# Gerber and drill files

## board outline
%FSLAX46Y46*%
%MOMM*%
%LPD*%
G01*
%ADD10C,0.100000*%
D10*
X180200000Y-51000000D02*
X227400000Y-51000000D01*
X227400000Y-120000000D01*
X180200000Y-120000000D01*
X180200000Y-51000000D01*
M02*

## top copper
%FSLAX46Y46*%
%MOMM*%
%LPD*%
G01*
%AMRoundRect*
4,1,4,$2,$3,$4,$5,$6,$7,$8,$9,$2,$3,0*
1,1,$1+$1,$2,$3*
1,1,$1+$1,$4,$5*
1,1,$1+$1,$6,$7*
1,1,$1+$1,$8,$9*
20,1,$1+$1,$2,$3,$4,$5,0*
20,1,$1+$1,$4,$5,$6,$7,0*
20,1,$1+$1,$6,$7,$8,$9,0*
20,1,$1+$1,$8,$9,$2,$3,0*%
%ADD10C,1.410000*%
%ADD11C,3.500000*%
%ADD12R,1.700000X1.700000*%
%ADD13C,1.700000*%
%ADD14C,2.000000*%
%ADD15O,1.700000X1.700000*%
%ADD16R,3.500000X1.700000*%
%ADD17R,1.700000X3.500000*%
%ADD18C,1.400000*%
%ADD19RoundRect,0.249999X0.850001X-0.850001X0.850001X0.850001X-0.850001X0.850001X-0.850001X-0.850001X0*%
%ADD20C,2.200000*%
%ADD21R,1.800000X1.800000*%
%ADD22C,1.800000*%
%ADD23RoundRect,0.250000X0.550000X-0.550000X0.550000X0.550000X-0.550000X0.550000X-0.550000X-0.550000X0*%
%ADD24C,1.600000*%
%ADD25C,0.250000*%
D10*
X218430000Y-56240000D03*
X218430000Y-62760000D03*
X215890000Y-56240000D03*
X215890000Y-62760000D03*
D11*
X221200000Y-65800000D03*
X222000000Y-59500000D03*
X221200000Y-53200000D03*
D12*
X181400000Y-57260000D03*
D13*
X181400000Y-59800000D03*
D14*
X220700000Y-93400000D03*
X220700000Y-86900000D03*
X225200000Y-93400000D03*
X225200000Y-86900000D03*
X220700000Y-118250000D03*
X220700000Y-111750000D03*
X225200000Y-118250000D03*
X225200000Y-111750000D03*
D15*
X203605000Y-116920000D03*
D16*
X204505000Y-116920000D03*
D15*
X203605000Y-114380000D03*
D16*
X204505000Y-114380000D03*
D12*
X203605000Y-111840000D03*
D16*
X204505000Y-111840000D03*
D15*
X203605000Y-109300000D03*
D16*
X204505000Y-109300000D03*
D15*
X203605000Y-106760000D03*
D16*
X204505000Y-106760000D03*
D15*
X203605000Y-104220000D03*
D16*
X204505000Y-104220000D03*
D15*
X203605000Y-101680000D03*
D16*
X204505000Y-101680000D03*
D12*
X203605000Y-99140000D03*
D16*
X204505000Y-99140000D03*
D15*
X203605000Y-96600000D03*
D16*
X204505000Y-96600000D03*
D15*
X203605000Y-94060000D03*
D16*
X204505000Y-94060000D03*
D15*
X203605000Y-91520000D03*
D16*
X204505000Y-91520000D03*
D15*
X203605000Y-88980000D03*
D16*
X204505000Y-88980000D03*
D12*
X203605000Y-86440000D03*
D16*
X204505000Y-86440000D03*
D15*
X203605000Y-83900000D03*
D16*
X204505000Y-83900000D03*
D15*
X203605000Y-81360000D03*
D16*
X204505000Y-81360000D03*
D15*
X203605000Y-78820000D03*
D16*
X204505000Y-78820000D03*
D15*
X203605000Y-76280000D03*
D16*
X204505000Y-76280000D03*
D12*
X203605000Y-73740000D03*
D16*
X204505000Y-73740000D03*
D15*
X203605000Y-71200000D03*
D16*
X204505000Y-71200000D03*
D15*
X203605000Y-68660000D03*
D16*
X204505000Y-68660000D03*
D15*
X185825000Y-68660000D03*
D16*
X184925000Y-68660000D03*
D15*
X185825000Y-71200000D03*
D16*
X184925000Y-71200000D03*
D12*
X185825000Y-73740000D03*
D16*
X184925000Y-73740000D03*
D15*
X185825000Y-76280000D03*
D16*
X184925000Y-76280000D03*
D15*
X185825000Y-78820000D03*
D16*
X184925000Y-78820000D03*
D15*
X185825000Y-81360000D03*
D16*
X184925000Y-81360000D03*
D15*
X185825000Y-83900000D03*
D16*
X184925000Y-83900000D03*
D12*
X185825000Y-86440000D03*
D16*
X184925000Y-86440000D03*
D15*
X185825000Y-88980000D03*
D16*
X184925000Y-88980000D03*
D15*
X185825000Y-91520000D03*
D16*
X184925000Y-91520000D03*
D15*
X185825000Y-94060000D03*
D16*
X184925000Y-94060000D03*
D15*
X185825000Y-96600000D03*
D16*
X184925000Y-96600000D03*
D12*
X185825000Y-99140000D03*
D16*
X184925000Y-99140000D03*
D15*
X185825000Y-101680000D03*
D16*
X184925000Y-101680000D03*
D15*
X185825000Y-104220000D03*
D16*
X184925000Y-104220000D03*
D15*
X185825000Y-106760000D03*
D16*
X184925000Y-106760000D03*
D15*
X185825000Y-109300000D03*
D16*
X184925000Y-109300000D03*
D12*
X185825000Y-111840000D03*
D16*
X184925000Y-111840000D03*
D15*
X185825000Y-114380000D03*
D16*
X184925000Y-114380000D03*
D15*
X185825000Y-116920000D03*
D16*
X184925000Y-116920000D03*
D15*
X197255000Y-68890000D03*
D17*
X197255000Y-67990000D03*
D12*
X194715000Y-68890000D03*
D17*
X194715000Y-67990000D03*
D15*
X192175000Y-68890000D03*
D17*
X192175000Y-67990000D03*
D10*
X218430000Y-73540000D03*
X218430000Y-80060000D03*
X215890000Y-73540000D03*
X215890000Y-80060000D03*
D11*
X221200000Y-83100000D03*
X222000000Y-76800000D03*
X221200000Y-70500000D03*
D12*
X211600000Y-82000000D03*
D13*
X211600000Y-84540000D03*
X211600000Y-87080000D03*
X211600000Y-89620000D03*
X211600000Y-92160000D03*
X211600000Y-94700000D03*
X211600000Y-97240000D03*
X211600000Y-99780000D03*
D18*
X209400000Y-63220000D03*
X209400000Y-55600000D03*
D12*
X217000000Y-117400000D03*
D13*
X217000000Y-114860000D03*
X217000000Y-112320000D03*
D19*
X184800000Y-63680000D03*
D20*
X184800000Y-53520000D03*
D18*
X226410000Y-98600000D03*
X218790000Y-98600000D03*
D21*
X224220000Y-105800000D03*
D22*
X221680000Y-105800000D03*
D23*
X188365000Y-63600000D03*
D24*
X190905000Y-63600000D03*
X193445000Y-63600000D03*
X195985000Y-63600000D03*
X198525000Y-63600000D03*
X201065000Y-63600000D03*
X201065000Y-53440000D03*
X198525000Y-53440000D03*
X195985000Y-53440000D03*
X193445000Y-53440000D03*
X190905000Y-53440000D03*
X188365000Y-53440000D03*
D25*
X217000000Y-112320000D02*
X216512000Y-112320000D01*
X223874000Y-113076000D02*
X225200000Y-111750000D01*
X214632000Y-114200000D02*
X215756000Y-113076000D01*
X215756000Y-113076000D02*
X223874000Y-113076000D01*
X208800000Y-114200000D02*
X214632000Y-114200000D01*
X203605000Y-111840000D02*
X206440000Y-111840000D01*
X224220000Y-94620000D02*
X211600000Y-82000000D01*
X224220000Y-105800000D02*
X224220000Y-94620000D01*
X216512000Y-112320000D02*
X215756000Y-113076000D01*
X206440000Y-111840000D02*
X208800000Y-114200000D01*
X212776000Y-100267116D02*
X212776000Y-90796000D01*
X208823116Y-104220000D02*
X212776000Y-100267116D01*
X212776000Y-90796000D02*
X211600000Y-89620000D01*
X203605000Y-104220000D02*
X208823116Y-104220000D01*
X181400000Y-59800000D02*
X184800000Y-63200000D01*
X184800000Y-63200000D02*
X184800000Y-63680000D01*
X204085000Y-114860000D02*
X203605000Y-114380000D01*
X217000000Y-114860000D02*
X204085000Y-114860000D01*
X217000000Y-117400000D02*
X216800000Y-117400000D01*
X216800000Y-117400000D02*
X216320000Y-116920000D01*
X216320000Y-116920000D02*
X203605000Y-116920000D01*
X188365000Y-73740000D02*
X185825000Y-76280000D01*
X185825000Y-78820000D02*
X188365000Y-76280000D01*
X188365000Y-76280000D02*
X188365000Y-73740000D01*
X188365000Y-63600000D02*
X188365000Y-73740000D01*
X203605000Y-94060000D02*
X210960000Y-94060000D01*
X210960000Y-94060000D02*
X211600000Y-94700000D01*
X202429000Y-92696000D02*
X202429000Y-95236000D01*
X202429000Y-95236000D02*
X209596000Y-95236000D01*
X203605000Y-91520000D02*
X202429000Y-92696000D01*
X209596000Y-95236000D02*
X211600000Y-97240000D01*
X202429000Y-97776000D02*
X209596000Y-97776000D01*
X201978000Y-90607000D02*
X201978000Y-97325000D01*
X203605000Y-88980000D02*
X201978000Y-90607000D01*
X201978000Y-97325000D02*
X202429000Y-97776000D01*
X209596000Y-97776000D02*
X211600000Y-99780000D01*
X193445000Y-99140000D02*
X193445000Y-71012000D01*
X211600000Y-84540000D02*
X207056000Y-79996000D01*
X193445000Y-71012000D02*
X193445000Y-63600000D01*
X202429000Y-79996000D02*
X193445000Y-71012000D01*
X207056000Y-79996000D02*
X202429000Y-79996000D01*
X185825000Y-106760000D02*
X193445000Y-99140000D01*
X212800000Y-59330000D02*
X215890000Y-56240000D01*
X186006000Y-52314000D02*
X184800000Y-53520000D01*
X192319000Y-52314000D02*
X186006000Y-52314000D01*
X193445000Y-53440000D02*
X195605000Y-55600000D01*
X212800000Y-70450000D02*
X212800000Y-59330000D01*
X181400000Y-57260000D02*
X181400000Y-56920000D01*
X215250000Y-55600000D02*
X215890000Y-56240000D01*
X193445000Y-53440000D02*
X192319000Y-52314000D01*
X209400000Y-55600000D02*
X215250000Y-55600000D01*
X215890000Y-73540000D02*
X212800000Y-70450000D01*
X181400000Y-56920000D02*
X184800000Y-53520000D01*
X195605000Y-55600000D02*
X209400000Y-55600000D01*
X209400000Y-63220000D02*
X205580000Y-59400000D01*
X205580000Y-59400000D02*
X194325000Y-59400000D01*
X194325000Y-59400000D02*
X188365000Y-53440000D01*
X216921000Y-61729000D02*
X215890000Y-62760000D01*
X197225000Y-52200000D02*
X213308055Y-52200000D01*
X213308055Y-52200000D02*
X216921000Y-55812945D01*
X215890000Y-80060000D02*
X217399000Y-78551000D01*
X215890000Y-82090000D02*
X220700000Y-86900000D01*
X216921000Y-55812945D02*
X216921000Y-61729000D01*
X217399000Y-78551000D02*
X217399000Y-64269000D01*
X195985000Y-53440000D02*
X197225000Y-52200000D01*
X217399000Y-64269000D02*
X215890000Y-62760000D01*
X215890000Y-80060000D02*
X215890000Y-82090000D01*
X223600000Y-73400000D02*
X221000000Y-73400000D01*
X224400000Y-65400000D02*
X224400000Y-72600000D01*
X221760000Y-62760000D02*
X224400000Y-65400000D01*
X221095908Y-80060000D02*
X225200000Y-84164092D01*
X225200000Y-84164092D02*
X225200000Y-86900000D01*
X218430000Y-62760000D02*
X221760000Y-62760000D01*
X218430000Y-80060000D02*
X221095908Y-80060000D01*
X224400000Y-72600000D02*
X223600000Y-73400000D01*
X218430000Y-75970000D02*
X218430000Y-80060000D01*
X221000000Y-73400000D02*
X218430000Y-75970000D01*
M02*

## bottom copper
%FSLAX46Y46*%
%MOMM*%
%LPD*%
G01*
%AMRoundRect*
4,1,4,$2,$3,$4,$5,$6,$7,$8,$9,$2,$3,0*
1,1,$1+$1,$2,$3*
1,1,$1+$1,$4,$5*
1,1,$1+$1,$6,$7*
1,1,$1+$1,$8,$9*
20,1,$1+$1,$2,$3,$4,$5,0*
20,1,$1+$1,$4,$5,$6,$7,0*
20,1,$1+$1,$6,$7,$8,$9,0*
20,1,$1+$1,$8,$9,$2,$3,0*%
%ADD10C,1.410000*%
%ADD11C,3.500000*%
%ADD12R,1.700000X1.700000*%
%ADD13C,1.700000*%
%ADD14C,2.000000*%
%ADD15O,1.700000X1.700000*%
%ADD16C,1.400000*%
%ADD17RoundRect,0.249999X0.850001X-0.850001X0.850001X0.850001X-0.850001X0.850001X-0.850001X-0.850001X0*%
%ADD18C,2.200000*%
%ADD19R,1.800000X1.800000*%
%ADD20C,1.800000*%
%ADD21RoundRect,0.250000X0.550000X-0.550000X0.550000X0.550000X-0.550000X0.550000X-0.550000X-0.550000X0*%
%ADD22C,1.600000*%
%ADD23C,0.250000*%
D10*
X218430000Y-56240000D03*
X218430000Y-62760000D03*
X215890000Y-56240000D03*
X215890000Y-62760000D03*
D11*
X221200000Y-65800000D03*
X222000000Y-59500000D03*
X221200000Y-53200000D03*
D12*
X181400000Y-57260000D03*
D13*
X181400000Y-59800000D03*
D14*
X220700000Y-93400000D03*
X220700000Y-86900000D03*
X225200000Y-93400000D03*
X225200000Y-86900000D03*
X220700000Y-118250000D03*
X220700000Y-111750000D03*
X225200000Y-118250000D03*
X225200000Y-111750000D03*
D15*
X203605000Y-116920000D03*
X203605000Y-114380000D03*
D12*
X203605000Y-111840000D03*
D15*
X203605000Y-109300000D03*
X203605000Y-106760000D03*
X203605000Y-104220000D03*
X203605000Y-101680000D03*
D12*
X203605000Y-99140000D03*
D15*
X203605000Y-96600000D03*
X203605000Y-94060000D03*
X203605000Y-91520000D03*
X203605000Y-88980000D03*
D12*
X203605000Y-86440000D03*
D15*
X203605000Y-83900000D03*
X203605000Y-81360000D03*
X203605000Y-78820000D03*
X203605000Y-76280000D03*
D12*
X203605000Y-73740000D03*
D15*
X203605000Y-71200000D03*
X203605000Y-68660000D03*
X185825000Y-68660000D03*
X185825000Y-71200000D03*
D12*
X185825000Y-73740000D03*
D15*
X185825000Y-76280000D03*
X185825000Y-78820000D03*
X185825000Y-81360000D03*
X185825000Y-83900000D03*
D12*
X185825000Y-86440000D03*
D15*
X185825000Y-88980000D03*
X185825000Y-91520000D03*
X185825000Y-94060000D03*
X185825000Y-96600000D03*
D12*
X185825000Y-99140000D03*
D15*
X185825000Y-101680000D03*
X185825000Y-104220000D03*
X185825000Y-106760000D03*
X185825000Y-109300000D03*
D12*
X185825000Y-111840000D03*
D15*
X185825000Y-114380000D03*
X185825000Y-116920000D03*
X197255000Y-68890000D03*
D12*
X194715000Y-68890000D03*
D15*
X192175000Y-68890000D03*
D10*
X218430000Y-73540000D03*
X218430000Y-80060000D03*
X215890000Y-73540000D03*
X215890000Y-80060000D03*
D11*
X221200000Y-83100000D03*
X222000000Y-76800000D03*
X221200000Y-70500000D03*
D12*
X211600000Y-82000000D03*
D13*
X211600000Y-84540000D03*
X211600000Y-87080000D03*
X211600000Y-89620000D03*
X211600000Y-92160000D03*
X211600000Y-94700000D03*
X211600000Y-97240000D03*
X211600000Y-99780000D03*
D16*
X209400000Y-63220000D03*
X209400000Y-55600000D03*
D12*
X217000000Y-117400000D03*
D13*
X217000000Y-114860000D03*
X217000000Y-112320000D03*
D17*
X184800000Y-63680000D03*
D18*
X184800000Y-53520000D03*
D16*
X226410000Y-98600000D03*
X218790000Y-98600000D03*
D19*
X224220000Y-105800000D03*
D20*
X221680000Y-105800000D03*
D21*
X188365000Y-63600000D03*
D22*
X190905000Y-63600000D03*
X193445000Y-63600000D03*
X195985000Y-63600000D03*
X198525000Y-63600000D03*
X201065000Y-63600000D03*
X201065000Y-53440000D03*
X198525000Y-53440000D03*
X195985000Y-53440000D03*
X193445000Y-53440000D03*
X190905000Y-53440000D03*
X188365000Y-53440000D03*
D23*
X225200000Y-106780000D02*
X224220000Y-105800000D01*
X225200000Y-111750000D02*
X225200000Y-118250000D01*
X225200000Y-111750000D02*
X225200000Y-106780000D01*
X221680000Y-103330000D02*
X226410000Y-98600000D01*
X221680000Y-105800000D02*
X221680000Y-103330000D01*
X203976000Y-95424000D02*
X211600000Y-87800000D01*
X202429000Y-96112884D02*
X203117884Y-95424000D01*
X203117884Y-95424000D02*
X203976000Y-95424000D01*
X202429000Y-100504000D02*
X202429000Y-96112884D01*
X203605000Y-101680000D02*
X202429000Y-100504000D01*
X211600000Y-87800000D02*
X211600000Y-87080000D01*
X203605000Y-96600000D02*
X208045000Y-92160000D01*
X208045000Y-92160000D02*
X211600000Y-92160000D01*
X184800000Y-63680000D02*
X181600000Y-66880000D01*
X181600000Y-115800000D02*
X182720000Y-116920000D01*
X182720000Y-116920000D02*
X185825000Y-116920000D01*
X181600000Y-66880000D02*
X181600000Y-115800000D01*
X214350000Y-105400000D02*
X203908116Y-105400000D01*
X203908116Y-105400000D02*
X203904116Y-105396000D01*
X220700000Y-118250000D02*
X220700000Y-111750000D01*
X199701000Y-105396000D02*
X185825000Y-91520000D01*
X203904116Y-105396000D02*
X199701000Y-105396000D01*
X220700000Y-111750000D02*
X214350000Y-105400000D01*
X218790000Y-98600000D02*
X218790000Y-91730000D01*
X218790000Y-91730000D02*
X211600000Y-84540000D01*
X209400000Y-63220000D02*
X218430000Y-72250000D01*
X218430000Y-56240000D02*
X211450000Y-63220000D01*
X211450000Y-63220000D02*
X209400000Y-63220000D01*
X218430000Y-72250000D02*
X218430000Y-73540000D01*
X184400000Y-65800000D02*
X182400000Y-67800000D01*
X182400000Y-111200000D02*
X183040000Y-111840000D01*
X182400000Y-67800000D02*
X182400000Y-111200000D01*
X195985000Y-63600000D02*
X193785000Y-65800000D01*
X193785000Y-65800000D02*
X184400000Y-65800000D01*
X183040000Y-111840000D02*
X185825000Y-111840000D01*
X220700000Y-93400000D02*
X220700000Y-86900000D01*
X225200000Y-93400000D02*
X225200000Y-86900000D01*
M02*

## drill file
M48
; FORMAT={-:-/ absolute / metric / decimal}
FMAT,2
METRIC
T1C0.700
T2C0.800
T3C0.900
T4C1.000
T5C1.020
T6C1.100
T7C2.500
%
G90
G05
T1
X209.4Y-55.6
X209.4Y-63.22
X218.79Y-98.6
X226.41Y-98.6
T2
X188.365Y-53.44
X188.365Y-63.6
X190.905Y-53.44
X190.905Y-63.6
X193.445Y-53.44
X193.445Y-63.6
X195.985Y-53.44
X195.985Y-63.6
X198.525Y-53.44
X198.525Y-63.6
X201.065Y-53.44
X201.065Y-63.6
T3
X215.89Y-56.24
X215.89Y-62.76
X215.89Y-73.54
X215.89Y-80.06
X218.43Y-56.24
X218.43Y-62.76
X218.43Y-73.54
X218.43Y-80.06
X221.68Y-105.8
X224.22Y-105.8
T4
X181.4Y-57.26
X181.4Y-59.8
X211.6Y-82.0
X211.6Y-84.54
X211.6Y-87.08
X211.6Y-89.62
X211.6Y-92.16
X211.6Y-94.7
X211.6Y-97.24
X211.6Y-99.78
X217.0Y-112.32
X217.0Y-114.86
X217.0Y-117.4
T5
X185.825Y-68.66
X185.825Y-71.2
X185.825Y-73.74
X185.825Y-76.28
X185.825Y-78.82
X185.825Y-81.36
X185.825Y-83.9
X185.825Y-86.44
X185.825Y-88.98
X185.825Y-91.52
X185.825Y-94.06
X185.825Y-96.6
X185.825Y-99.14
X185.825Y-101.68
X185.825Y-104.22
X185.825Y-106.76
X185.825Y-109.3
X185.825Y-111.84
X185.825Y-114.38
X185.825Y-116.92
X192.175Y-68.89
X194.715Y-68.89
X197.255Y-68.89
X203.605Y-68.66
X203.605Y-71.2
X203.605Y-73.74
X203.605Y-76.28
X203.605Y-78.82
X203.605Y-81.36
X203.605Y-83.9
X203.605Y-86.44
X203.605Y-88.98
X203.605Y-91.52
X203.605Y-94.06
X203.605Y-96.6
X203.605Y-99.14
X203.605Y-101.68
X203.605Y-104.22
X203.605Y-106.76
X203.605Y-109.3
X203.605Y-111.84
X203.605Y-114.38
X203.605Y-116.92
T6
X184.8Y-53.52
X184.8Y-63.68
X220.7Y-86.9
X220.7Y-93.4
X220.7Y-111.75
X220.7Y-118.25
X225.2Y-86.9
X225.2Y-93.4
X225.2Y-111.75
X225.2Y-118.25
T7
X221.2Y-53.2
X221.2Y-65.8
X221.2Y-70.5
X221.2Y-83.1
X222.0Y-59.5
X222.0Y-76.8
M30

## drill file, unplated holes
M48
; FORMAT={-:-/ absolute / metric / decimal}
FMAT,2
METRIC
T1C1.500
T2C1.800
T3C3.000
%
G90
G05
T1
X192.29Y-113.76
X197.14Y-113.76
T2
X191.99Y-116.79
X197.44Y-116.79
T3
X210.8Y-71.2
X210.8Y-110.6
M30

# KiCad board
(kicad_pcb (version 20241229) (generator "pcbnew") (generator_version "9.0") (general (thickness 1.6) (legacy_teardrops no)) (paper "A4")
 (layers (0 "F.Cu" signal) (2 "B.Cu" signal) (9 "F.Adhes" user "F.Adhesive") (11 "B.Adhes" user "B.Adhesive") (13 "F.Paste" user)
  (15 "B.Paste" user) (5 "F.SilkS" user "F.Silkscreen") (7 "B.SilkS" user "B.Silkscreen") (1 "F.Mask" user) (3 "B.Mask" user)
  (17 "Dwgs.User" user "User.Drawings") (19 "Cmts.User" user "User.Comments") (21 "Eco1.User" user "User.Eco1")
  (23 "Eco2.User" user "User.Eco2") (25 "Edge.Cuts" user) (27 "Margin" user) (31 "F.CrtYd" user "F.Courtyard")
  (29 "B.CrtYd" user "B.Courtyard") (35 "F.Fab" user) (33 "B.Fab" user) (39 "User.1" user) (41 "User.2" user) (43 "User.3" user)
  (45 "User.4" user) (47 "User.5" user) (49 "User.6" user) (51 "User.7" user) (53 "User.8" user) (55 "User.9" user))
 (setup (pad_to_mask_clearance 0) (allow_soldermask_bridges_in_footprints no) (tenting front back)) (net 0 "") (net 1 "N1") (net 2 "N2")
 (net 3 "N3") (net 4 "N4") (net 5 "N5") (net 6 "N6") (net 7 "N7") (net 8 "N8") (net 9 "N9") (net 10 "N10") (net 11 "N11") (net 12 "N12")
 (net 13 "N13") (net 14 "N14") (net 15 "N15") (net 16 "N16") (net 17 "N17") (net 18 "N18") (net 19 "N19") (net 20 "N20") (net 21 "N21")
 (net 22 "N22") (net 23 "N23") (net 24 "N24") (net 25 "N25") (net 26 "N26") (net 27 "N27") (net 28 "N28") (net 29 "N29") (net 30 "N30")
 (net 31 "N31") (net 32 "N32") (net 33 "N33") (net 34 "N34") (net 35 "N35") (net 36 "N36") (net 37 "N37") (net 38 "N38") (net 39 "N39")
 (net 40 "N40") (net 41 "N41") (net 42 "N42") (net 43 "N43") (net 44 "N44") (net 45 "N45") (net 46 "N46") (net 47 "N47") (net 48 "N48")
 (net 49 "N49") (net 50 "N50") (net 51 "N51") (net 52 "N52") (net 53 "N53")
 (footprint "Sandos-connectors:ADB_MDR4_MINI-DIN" (layer "F.Cu") (at 220.2 59.5 90)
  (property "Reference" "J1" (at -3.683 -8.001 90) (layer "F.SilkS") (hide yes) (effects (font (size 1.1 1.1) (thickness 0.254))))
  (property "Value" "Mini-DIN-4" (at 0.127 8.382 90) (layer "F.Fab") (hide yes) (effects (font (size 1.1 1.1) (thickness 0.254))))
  (pad "1" thru_hole circle (at 3.26 -1.77 90) (size 1.41 1.41) (drill 0.9) (layers "*.Cu" "*.Mask") (remove_unused_layers no) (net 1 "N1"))
  (pad "2" thru_hole circle (at -3.26 -1.77 90) (size 1.41 1.41) (drill 0.9) (layers "*.Cu" "*.Mask") (remove_unused_layers no) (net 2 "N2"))
  (pad "3" thru_hole circle (at 3.26 -4.31 90) (size 1.41 1.41) (drill 0.9) (layers "*.Cu" "*.Mask") (remove_unused_layers no) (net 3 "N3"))
  (pad "4" thru_hole circle (at -3.26 -4.31 90) (size 1.41 1.41) (drill 0.9) (layers "*.Cu" "*.Mask") (remove_unused_layers no) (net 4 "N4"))
  (pad "9" thru_hole circle (at -6.3 1 90) (size 3.5 3.5) (drill 2.5) (layers "*.Cu" "*.Mask") (remove_unused_layers no))
  (pad "9" thru_hole circle (at 0 1.8 90) (size 3.5 3.5) (drill 2.5) (layers "*.Cu" "*.Mask") (remove_unused_layers no))
  (pad "9" thru_hole circle (at 6.3 1 90) (size 3.5 3.5) (drill 2.5) (layers "*.Cu" "*.Mask") (remove_unused_layers no)))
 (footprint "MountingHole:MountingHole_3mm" (layer "F.Cu") (at 210.8 110.6)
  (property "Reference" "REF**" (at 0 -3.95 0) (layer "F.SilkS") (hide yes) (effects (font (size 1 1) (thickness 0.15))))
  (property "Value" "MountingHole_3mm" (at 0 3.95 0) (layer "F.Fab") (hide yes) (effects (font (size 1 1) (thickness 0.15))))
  (pad "" np_thru_hole circle (at 0 0) (size 3 3) (drill 3) (layers "*.Cu" "*.Mask")))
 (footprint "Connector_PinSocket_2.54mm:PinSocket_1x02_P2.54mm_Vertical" (layer "F.Cu") (at 181.4 57.26)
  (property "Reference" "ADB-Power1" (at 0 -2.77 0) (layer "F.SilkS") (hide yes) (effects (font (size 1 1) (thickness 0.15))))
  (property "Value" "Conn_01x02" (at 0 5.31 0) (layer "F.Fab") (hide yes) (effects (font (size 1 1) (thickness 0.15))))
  (pad "1" thru_hole rect (at 0 0) (size 1.7 1.7) (drill 1) (layers "*.Cu" "*.Mask") (remove_unused_layers no) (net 3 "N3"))
  (pad "2" thru_hole circle (at 0 2.54) (size 1.7 1.7) (drill 1) (layers "*.Cu" "*.Mask") (remove_unused_layers no) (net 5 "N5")))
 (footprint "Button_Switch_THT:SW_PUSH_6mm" (layer "F.Cu") (at 220.7 93.4 90)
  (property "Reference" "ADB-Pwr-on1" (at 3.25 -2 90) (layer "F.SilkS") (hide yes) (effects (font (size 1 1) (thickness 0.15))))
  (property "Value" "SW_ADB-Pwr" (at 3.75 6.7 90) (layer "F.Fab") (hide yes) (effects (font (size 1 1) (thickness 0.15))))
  (pad "1" thru_hole circle (at 0 0 180) (size 2 2) (drill 1.1) (layers "*.Cu" "*.Mask") (remove_unused_layers no) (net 4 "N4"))
  (pad "1" thru_hole circle (at 6.5 0 180) (size 2 2) (drill 1.1) (layers "*.Cu" "*.Mask") (remove_unused_layers no) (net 4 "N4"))
  (pad "2" thru_hole circle (at 0 4.5 180) (size 2 2) (drill 1.1) (layers "*.Cu" "*.Mask") (remove_unused_layers no) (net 2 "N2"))
  (pad "2" thru_hole circle (at 6.5 4.5 180) (size 2 2) (drill 1.1) (layers "*.Cu" "*.Mask") (remove_unused_layers no) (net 2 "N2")))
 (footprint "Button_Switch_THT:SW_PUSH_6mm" (layer "F.Cu") (at 220.7 118.25 90)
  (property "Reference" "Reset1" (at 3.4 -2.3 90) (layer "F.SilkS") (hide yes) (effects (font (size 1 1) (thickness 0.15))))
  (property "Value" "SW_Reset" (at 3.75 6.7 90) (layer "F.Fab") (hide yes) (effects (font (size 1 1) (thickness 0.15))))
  (pad "1" thru_hole circle (at 0 0 180) (size 2 2) (drill 1.1) (layers "*.Cu" "*.Mask") (remove_unused_layers no) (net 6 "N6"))
  (pad "1" thru_hole circle (at 6.5 0 180) (size 2 2) (drill 1.1) (layers "*.Cu" "*.Mask") (remove_unused_layers no) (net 6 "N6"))
  (pad "2" thru_hole circle (at 0 4.5 180) (size 2 2) (drill 1.1) (layers "*.Cu" "*.Mask") (remove_unused_layers no) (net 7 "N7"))
  (pad "2" thru_hole circle (at 6.5 4.5 180) (size 2 2) (drill 1.1) (layers "*.Cu" "*.Mask") (remove_unused_layers no) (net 7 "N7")))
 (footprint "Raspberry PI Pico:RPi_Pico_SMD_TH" (layer "F.Cu") (at 194.715 92.79 180)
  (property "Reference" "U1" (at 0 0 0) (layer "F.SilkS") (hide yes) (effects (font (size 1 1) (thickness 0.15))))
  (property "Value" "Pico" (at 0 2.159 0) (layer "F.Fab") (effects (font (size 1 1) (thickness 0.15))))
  (pad "" np_thru_hole oval (at -2.725 -24 180) (size 1.8 1.8) (drill 1.8) (layers "*.Cu" "*.Mask"))
  (pad "" np_thru_hole oval (at -2.425 -20.97 180) (size 1.5 1.5) (drill 1.5) (layers "*.Cu" "*.Mask"))
  (pad "" np_thru_hole oval (at 2.425 -20.97 180) (size 1.5 1.5) (drill 1.5) (layers "*.Cu" "*.Mask"))
  (pad "" np_thru_hole oval (at 2.725 -24 180) (size 1.8 1.8) (drill 1.8) (layers "*.Cu" "*.Mask"))
  (pad "1" thru_hole oval (at -8.89 -24.13 180) (size 1.7 1.7) (drill 1.02) (layers "*.Cu" "*.Mask") (remove_unused_layers no) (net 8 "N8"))
  (pad "1" smd rect (at -8.89 -24.13 180) (size 3.5 1.7) (drill (offset -0.9 0)) (layers "F.Cu" "F.Mask") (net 8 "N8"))
  (pad "2" thru_hole oval (at -8.89 -21.59 180) (size 1.7 1.7) (drill 1.02) (layers "*.Cu" "*.Mask") (remove_unused_layers no) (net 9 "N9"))
  (pad "2" smd rect (at -8.89 -21.59 180) (size 3.5 1.7) (drill (offset -0.9 0)) (layers "F.Cu" "F.Mask") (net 9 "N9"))
  (pad "3" thru_hole rect (at -8.89 -19.05 180) (size 1.7 1.7) (drill 1.02) (layers "*.Cu" "*.Mask") (remove_unused_layers no) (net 7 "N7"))
  (pad "3" smd rect (at -8.89 -19.05 180) (size 3.5 1.7) (drill (offset -0.9 0)) (layers "F.Cu" "F.Mask") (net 7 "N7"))
  (pad "4" thru_hole oval (at -8.89 -16.51 180) (size 1.7 1.7) (drill 1.02) (layers "*.Cu" "*.Mask") (remove_unused_layers no)
   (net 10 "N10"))
  (pad "4" smd rect (at -8.89 -16.51 180) (size 3.5 1.7) (drill (offset -0.9 0)) (layers "F.Cu" "F.Mask") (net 10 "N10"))
  (pad "5" thru_hole oval (at -8.89 -13.97 180) (size 1.7 1.7) (drill 1.02) (layers "*.Cu" "*.Mask") (remove_unused_layers no)
   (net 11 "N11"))
  (pad "5" smd rect (at -8.89 -13.97 180) (size 3.5 1.7) (drill (offset -0.9 0)) (layers "F.Cu" "F.Mask") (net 11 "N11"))
  (pad "6" thru_hole oval (at -8.89 -11.43 180) (size 1.7 1.7) (drill 1.02) (layers "*.Cu" "*.Mask") (remove_unused_layers no)
   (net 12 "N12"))
  (pad "6" smd rect (at -8.89 -11.43 180) (size 3.5 1.7) (drill (offset -0.9 0)) (layers "F.Cu" "F.Mask") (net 12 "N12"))
  (pad "7" thru_hole oval (at -8.89 -8.89 180) (size 1.7 1.7) (drill 1.02) (layers "*.Cu" "*.Mask") (remove_unused_layers no) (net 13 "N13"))
  (pad "7" smd rect (at -8.89 -8.89 180) (size 3.5 1.7) (drill (offset -0.9 0)) (layers "F.Cu" "F.Mask") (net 13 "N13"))
  (pad "8" thru_hole rect (at -8.89 -6.35 180) (size 1.7 1.7) (drill 1.02) (layers "*.Cu" "*.Mask") (remove_unused_layers no) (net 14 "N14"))
  (pad "8" smd rect (at -8.89 -6.35 180) (size 3.5 1.7) (drill (offset -0.9 0)) (layers "F.Cu" "F.Mask") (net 14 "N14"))
  (pad "9" thru_hole oval (at -8.89 -3.81 180) (size 1.7 1.7) (drill 1.02) (layers "*.Cu" "*.Mask") (remove_unused_layers no) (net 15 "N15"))
  (pad "9" smd rect (at -8.89 -3.81 180) (size 3.5 1.7) (drill (offset -0.9 0)) (layers "F.Cu" "F.Mask") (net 15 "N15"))
  (pad "10" thru_hole oval (at -8.89 -1.27 180) (size 1.7 1.7) (drill 1.02) (layers "*.Cu" "*.Mask") (remove_unused_layers no)
   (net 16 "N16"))
  (pad "10" smd rect (at -8.89 -1.27 180) (size 3.5 1.7) (drill (offset -0.9 0)) (layers "F.Cu" "F.Mask") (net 16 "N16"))
  (pad "11" thru_hole oval (at -8.89 1.27 180) (size 1.7 1.7) (drill 1.02) (layers "*.Cu" "*.Mask") (remove_unused_layers no) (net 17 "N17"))
  (pad "11" smd rect (at -8.89 1.27 180) (size 3.5 1.7) (drill (offset -0.9 0)) (layers "F.Cu" "F.Mask") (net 17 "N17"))
  (pad "12" thru_hole oval (at -8.89 3.81 180) (size 1.7 1.7) (drill 1.02) (layers "*.Cu" "*.Mask") (remove_unused_layers no) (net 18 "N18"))
  (pad "12" smd rect (at -8.89 3.81 180) (size 3.5 1.7) (drill (offset -0.9 0)) (layers "F.Cu" "F.Mask") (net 18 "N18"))
  (pad "13" thru_hole rect (at -8.89 6.35 180) (size 1.7 1.7) (drill 1.02) (layers "*.Cu" "*.Mask") (remove_unused_layers no) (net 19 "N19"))
  (pad "13" smd rect (at -8.89 6.35 180) (size 3.5 1.7) (drill (offset -0.9 0)) (layers "F.Cu" "F.Mask") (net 19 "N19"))
  (pad "14" thru_hole oval (at -8.89 8.89 180) (size 1.7 1.7) (drill 1.02) (layers "*.Cu" "*.Mask") (remove_unused_layers no) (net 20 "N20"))
  (pad "14" smd rect (at -8.89 8.89 180) (size 3.5 1.7) (drill (offset -0.9 0)) (layers "F.Cu" "F.Mask") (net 20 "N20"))
  (pad "15" thru_hole oval (at -8.89 11.43 180) (size 1.7 1.7) (drill 1.02) (layers "*.Cu" "*.Mask") (remove_unused_layers no)
   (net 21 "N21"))
  (pad "15" smd rect (at -8.89 11.43 180) (size 3.5 1.7) (drill (offset -0.9 0)) (layers "F.Cu" "F.Mask") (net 21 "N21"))
  (pad "16" thru_hole oval (at -8.89 13.97 180) (size 1.7 1.7) (drill 1.02) (layers "*.Cu" "*.Mask") (remove_unused_layers no)
   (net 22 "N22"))
  (pad "16" smd rect (at -8.89 13.97 180) (size 3.5 1.7) (drill (offset -0.9 0)) (layers "F.Cu" "F.Mask") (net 22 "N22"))
  (pad "17" thru_hole oval (at -8.89 16.51 180) (size 1.7 1.7) (drill 1.02) (layers "*.Cu" "*.Mask") (remove_unused_layers no)
   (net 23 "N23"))
  (pad "17" smd rect (at -8.89 16.51 180) (size 3.5 1.7) (drill (offset -0.9 0)) (layers "F.Cu" "F.Mask") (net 23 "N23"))
  (pad "18" thru_hole rect (at -8.89 19.05 180) (size 1.7 1.7) (drill 1.02) (layers "*.Cu" "*.Mask") (remove_unused_layers no)
   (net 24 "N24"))
  (pad "18" smd rect (at -8.89 19.05 180) (size 3.5 1.7) (drill (offset -0.9 0)) (layers "F.Cu" "F.Mask") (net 24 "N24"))
  (pad "19" thru_hole oval (at -8.89 21.59 180) (size 1.7 1.7) (drill 1.02) (layers "*.Cu" "*.Mask") (remove_unused_layers no)
   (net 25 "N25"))
  (pad "19" smd rect (at -8.89 21.59 180) (size 3.5 1.7) (drill (offset -0.9 0)) (layers "F.Cu" "F.Mask") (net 25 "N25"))
  (pad "20" thru_hole oval (at -8.89 24.13 180) (size 1.7 1.7) (drill 1.02) (layers "*.Cu" "*.Mask") (remove_unused_layers no)
   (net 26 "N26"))
  (pad "20" smd rect (at -8.89 24.13 180) (size 3.5 1.7) (drill (offset -0.9 0)) (layers "F.Cu" "F.Mask") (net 26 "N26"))
  (pad "21" thru_hole oval (at 8.89 24.13 180) (size 1.7 1.7) (drill 1.02) (layers "*.Cu" "*.Mask") (remove_unused_layers no) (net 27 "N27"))
  (pad "21" smd rect (at 8.89 24.13 180) (size 3.5 1.7) (drill (offset 0.9 0)) (layers "F.Cu" "F.Mask") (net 27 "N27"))
  (pad "22" thru_hole oval (at 8.89 21.59 180) (size 1.7 1.7) (drill 1.02) (layers "*.Cu" "*.Mask") (remove_unused_layers no) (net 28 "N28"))
  (pad "22" smd rect (at 8.89 21.59 180) (size 3.5 1.7) (drill (offset 0.9 0)) (layers "F.Cu" "F.Mask") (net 28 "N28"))
  (pad "23" thru_hole rect (at 8.89 19.05 180) (size 1.7 1.7) (drill 1.02) (layers "*.Cu" "*.Mask") (remove_unused_layers no) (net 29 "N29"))
  (pad "23" smd rect (at 8.89 19.05 180) (size 3.5 1.7) (drill (offset 0.9 0)) (layers "F.Cu" "F.Mask") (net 29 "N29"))
  (pad "24" thru_hole oval (at 8.89 16.51 180) (size 1.7 1.7) (drill 1.02) (layers "*.Cu" "*.Mask") (remove_unused_layers no) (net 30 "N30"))
  (pad "24" smd rect (at 8.89 16.51 180) (size 3.5 1.7) (drill (offset 0.9 0)) (layers "F.Cu" "F.Mask") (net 30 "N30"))
  (pad "25" thru_hole oval (at 8.89 13.97 180) (size 1.7 1.7) (drill 1.02) (layers "*.Cu" "*.Mask") (remove_unused_layers no) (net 30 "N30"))
  (pad "25" smd rect (at 8.89 13.97 180) (size 3.5 1.7) (drill (offset 0.9 0)) (layers "F.Cu" "F.Mask") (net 30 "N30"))
  (pad "26" thru_hole oval (at 8.89 11.43 180) (size 1.7 1.7) (drill 1.02) (layers "*.Cu" "*.Mask") (remove_unused_layers no) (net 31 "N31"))
  (pad "26" smd rect (at 8.89 11.43 180) (size 3.5 1.7) (drill (offset 0.9 0)) (layers "F.Cu" "F.Mask") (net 31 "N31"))
  (pad "27" thru_hole oval (at 8.89 8.89 180) (size 1.7 1.7) (drill 1.02) (layers "*.Cu" "*.Mask") (remove_unused_layers no) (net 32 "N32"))
  (pad "27" smd rect (at 8.89 8.89 180) (size 3.5 1.7) (drill (offset 0.9 0)) (layers "F.Cu" "F.Mask") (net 32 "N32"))
  (pad "28" thru_hole rect (at 8.89 6.35 180) (size 1.7 1.7) (drill 1.02) (layers "*.Cu" "*.Mask") (remove_unused_layers no) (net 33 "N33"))
  (pad "28" smd rect (at 8.89 6.35 180) (size 3.5 1.7) (drill (offset 0.9 0)) (layers "F.Cu" "F.Mask") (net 33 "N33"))
  (pad "29" thru_hole oval (at 8.89 3.81 180) (size 1.7 1.7) (drill 1.02) (layers "*.Cu" "*.Mask") (remove_unused_layers no) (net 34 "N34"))
  (pad "29" smd rect (at 8.89 3.81 180) (size 3.5 1.7) (drill (offset 0.9 0)) (layers "F.Cu" "F.Mask") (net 34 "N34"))
  (pad "30" thru_hole oval (at 8.89 1.27 180) (size 1.7 1.7) (drill 1.02) (layers "*.Cu" "*.Mask") (remove_unused_layers no) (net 6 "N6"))
  (pad "30" smd rect (at 8.89 1.27 180) (size 3.5 1.7) (drill (offset 0.9 0)) (layers "F.Cu" "F.Mask") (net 6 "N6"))
  (pad "31" thru_hole oval (at 8.89 -1.27 180) (size 1.7 1.7) (drill 1.02) (layers "*.Cu" "*.Mask") (remove_unused_layers no) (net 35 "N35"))
  (pad "31" smd rect (at 8.89 -1.27 180) (size 3.5 1.7) (drill (offset 0.9 0)) (layers "F.Cu" "F.Mask") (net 35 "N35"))
  (pad "32" thru_hole oval (at 8.89 -3.81 180) (size 1.7 1.7) (drill 1.02) (layers "*.Cu" "*.Mask") (remove_unused_layers no) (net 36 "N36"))
  (pad "32" smd rect (at 8.89 -3.81 180) (size 3.5 1.7) (drill (offset 0.9 0)) (layers "F.Cu" "F.Mask") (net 36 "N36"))
  (pad "33" thru_hole rect (at 8.89 -6.35 180) (size 1.7 1.7) (drill 1.02) (layers "*.Cu" "*.Mask") (remove_unused_layers no) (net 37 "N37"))
  (pad "33" smd rect (at 8.89 -6.35 180) (size 3.5 1.7) (drill (offset 0.9 0)) (layers "F.Cu" "F.Mask") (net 37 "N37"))
  (pad "34" thru_hole oval (at 8.89 -8.89 180) (size 1.7 1.7) (drill 1.02) (layers "*.Cu" "*.Mask") (remove_unused_layers no) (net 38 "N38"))
  (pad "34" smd rect (at 8.89 -8.89 180) (size 3.5 1.7) (drill (offset 0.9 0)) (layers "F.Cu" "F.Mask") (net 38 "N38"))
  (pad "35" thru_hole oval (at 8.89 -11.43 180) (size 1.7 1.7) (drill 1.02) (layers "*.Cu" "*.Mask") (remove_unused_layers no)
   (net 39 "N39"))
  (pad "35" smd rect (at 8.89 -11.43 180) (size 3.5 1.7) (drill (offset 0.9 0)) (layers "F.Cu" "F.Mask") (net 39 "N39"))
  (pad "36" thru_hole oval (at 8.89 -13.97 180) (size 1.7 1.7) (drill 1.02) (layers "*.Cu" "*.Mask") (remove_unused_layers no)
   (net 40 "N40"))
  (pad "36" smd rect (at 8.89 -13.97 180) (size 3.5 1.7) (drill (offset 0.9 0)) (layers "F.Cu" "F.Mask") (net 40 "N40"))
  (pad "37" thru_hole oval (at 8.89 -16.51 180) (size 1.7 1.7) (drill 1.02) (layers "*.Cu" "*.Mask") (remove_unused_layers no)
   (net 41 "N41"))
  (pad "37" smd rect (at 8.89 -16.51 180) (size 3.5 1.7) (drill (offset 0.9 0)) (layers "F.Cu" "F.Mask") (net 41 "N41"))
  (pad "38" thru_hole rect (at 8.89 -19.05 180) (size 1.7 1.7) (drill 1.02) (layers "*.Cu" "*.Mask") (remove_unused_layers no)
   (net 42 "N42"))
  (pad "38" smd rect (at 8.89 -19.05 180) (size 3.5 1.7) (drill (offset 0.9 0)) (layers "F.Cu" "F.Mask") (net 42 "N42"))
  (pad "39" thru_hole oval (at 8.89 -21.59 180) (size 1.7 1.7) (drill 1.02) (layers "*.Cu" "*.Mask") (remove_unused_layers no)
   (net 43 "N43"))
  (pad "39" smd rect (at 8.89 -21.59 180) (size 3.5 1.7) (drill (offset 0.9 0)) (layers "F.Cu" "F.Mask") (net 43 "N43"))
  (pad "40" thru_hole oval (at 8.89 -24.13 180) (size 1.7 1.7) (drill 1.02) (layers "*.Cu" "*.Mask") (remove_unused_layers no) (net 5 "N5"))
  (pad "40" smd rect (at 8.89 -24.13 180) (size 3.5 1.7) (drill (offset 0.9 0)) (layers "F.Cu" "F.Mask") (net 5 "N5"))
  (pad "41" thru_hole oval (at -2.54 23.9 180) (size 1.7 1.7) (drill 1.02) (layers "*.Cu" "*.Mask") (remove_unused_layers no) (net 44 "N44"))
  (pad "41" smd rect (at -2.54 23.9 270) (size 3.5 1.7) (drill (offset -0.9 0)) (layers "F.Cu" "F.Mask") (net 44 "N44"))
  (pad "42" thru_hole rect (at 0 23.9 180) (size 1.7 1.7) (drill 1.02) (layers "*.Cu" "*.Mask") (remove_unused_layers no) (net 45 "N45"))
  (pad "42" smd rect (at 0 23.9 270) (size 3.5 1.7) (drill (offset -0.9 0)) (layers "F.Cu" "F.Mask") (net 45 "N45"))
  (pad "43" thru_hole oval (at 2.54 23.9 180) (size 1.7 1.7) (drill 1.02) (layers "*.Cu" "*.Mask") (remove_unused_layers no) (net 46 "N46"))
  (pad "43" smd rect (at 2.54 23.9 270) (size 3.5 1.7) (drill (offset -0.9 0)) (layers "F.Cu" "F.Mask") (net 46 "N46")))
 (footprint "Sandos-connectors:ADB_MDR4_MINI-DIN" (layer "F.Cu") (at 220.2 76.8 90)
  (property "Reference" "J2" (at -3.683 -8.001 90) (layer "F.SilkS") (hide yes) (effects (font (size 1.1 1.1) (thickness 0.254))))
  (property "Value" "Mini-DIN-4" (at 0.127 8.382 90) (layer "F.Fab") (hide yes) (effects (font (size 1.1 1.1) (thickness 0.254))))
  (pad "1" thru_hole circle (at 3.26 -1.77 90) (size 1.41 1.41) (drill 0.9) (layers "*.Cu" "*.Mask") (remove_unused_layers no) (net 1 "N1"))
  (pad "2" thru_hole circle (at -3.26 -1.77 90) (size 1.41 1.41) (drill 0.9) (layers "*.Cu" "*.Mask") (remove_unused_layers no) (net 2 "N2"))
  (pad "3" thru_hole circle (at 3.26 -4.31 90) (size 1.41 1.41) (drill 0.9) (layers "*.Cu" "*.Mask") (remove_unused_layers no) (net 3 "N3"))
  (pad "4" thru_hole circle (at -3.26 -4.31 90) (size 1.41 1.41) (drill 0.9) (layers "*.Cu" "*.Mask") (remove_unused_layers no) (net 4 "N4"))
  (pad "9" thru_hole circle (at -6.3 1 90) (size 3.5 3.5) (drill 2.5) (layers "*.Cu" "*.Mask") (remove_unused_layers no))
  (pad "9" thru_hole circle (at 0 1.8 90) (size 3.5 3.5) (drill 2.5) (layers "*.Cu" "*.Mask") (remove_unused_layers no))
  (pad "9" thru_hole circle (at 6.3 1 90) (size 3.5 3.5) (drill 2.5) (layers "*.Cu" "*.Mask") (remove_unused_layers no)))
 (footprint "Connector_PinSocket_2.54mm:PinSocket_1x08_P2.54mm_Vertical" (layer "F.Cu") (at 211.6 82)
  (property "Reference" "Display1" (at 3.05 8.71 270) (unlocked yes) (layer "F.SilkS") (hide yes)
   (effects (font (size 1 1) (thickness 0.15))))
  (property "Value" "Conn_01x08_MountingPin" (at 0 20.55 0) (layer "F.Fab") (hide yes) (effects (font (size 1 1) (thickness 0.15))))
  (pad "1" thru_hole rect (at 0 0) (size 1.7 1.7) (drill 1) (layers "*.Cu" "*.Mask") (remove_unused_layers no) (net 7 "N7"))
  (pad "2" thru_hole circle (at 0 2.54) (size 1.7 1.7) (drill 1) (layers "*.Cu" "*.Mask") (remove_unused_layers no) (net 40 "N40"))
  (pad "3" thru_hole circle (at 0 5.08) (size 1.7 1.7) (drill 1) (layers "*.Cu" "*.Mask") (remove_unused_layers no) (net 13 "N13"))
  (pad "4" thru_hole circle (at 0 7.62) (size 1.7 1.7) (drill 1) (layers "*.Cu" "*.Mask") (remove_unused_layers no) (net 12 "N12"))
  (pad "5" thru_hole circle (at 0 10.16) (size 1.7 1.7) (drill 1) (layers "*.Cu" "*.Mask") (remove_unused_layers no) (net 15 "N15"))
  (pad "6" thru_hole circle (at 0 12.7) (size 1.7 1.7) (drill 1) (layers "*.Cu" "*.Mask") (remove_unused_layers no) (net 16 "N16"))
  (pad "7" thru_hole circle (at 0 15.24) (size 1.7 1.7) (drill 1) (layers "*.Cu" "*.Mask") (remove_unused_layers no) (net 17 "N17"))
  (pad "8" thru_hole circle (at 0 17.78) (size 1.7 1.7) (drill 1) (layers "*.Cu" "*.Mask") (remove_unused_layers no) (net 18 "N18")))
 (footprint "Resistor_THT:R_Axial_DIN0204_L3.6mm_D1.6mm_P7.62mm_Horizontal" (layer "F.Cu") (at 209.4 63.22 90)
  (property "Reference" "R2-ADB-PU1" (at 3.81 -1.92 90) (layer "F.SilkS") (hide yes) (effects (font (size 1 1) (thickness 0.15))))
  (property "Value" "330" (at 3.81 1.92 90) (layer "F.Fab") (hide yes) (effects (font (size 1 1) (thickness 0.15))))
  (pad "1" thru_hole circle (at 0 0 90) (size 1.4 1.4) (drill 0.7) (layers "*.Cu" "*.Mask") (remove_unused_layers no) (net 1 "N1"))
  (pad "2" thru_hole circle (at 7.62 0 90) (size 1.4 1.4) (drill 0.7) (layers "*.Cu" "*.Mask") (remove_unused_layers no) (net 3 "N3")))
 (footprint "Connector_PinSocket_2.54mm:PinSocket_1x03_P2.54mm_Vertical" (layer "F.Cu") (at 217 117.4 180)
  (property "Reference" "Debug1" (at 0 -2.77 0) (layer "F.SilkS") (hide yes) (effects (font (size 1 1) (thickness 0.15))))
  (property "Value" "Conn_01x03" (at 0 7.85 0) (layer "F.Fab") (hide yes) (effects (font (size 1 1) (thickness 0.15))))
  (pad "1" thru_hole rect (at 0 0 180) (size 1.7 1.7) (drill 1) (layers "*.Cu" "*.Mask") (remove_unused_layers no) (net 8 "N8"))
  (pad "2" thru_hole circle (at 0 2.54 180) (size 1.7 1.7) (drill 1) (layers "*.Cu" "*.Mask") (remove_unused_layers no) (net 9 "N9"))
  (pad "3" thru_hole circle (at 0 5.08 180) (size 1.7 1.7) (drill 1) (layers "*.Cu" "*.Mask") (remove_unused_layers no) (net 7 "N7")))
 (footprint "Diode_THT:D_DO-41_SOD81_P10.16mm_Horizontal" (layer "F.Cu") (at 184.8 63.68 90)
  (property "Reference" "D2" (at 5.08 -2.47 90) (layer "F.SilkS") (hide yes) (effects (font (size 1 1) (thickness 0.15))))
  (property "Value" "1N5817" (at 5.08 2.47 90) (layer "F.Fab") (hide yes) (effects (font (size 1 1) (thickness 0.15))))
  (pad "1" thru_hole roundrect (at 0 0 90) (size 2.2 2.2) (drill 1.1) (layers "*.Cu" "*.Mask") (remove_unused_layers no)
   (roundrect_rratio 0.113636) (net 5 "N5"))
  (pad "2" thru_hole circle (at 10.16 0 90) (size 2.2 2.2) (drill 1.1) (layers "*.Cu" "*.Mask") (remove_unused_layers no) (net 3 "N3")))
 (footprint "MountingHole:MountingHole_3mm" (layer "F.Cu") (at 210.8 71.2)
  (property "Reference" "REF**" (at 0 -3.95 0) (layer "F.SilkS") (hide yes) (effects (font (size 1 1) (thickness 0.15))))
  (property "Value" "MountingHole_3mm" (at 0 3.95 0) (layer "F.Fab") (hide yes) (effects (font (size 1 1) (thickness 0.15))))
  (pad "" np_thru_hole circle (at 0 0) (size 3 3) (drill 3) (layers "*.Cu" "*.Mask")))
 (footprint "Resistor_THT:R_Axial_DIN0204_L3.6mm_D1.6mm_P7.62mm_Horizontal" (layer "F.Cu") (at 226.41 98.6 180)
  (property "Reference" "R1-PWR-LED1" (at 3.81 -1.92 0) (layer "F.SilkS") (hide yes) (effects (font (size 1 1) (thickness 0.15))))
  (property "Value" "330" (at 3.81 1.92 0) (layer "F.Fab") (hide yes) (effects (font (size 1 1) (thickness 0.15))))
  (pad "1" thru_hole circle (at 0 0 180) (size 1.4 1.4) (drill 0.7) (layers "*.Cu" "*.Mask") (remove_unused_layers no) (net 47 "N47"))
  (pad "2" thru_hole circle (at 7.62 0 180) (size 1.4 1.4) (drill 0.7) (layers "*.Cu" "*.Mask") (remove_unused_layers no) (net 40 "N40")))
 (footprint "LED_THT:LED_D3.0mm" (layer "F.Cu") (at 224.22 105.8 180)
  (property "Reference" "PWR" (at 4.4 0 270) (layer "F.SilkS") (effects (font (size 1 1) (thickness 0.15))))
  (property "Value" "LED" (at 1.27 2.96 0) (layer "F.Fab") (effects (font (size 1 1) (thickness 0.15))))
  (pad "1" thru_hole rect (at 0 0 180) (size 1.8 1.8) (drill 0.9) (layers "*.Cu" "*.Mask") (remove_unused_layers no) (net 7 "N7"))
  (pad "2" thru_hole circle (at 2.54 0 180) (size 1.8 1.8) (drill 0.9) (layers "*.Cu" "*.Mask") (remove_unused_layers no) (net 47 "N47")))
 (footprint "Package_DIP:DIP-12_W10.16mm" (layer "F.Cu") (at 188.365 63.6 90)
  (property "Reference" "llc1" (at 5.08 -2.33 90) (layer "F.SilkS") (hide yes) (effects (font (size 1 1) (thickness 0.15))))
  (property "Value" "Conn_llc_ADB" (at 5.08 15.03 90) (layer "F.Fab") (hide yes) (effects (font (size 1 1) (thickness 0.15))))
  (pad "1" thru_hole roundrect (at 0 0 90) (size 1.6 1.6) (drill 0.8) (layers "*.Cu" "*.Mask") (remove_unused_layers no)
   (roundrect_rratio 0.15625) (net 30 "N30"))
  (pad "2" thru_hole circle (at 0 2.54 90) (size 1.6 1.6) (drill 0.8) (layers "*.Cu" "*.Mask") (remove_unused_layers no) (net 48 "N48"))
  (pad "3" thru_hole circle (at 0 5.08 90) (size 1.6 1.6) (drill 0.8) (layers "*.Cu" "*.Mask") (remove_unused_layers no) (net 40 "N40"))
  (pad "4" thru_hole circle (at 0 7.62 90) (size 1.6 1.6) (drill 0.8) (layers "*.Cu" "*.Mask") (remove_unused_layers no) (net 42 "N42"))
  (pad "5" thru_hole circle (at 0 10.16 90) (size 1.6 1.6) (drill 0.8) (layers "*.Cu" "*.Mask") (remove_unused_layers no) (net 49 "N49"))
  (pad "6" thru_hole circle (at 0 12.7 90) (size 1.6 1.6) (drill 0.8) (layers "*.Cu" "*.Mask") (remove_unused_layers no) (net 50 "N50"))
  (pad "7" thru_hole circle (at 10.16 12.7 90) (size 1.6 1.6) (drill 0.8) (layers "*.Cu" "*.Mask") (remove_unused_layers no) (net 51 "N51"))
  (pad "8" thru_hole circle (at 10.16 10.16 90) (size 1.6 1.6) (drill 0.8) (layers "*.Cu" "*.Mask") (remove_unused_layers no) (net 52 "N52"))
  (pad "9" thru_hole circle (at 10.16 7.62 90) (size 1.6 1.6) (drill 0.8) (layers "*.Cu" "*.Mask") (remove_unused_layers no) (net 4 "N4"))
  (pad "10" thru_hole circle (at 10.16 5.08 90) (size 1.6 1.6) (drill 0.8) (layers "*.Cu" "*.Mask") (remove_unused_layers no) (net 3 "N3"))
  (pad "11" thru_hole circle (at 10.16 2.54 90) (size 1.6 1.6) (drill 0.8) (layers "*.Cu" "*.Mask") (remove_unused_layers no) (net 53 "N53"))
  (pad "12" thru_hole circle (at 10.16 0 90) (size 1.6 1.6) (drill 0.8) (layers "*.Cu" "*.Mask") (remove_unused_layers no) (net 1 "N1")))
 (gr_rect (start 180.2 51) (end 227.4 120) (stroke (width 0.1) (type solid)) (fill no) (layer "Edge.Cuts"))
 (segment (start 217 112.32) (end 216.512 112.32) (width 0.25) (layer "F.Cu") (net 7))
 (segment (start 223.874 113.076) (end 225.2 111.75) (width 0.25) (layer "F.Cu") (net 7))
 (segment (start 214.632 114.2) (end 215.756 113.076) (width 0.25) (layer "F.Cu") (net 7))
 (segment (start 215.756 113.076) (end 223.874 113.076) (width 0.25) (layer "F.Cu") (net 7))
 (segment (start 208.8 114.2) (end 214.632 114.2) (width 0.25) (layer "F.Cu") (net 7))
 (segment (start 203.605 111.84) (end 206.44 111.84) (width 0.25) (layer "F.Cu") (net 7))
 (segment (start 224.22 94.62) (end 211.6 82) (width 0.25) (layer "F.Cu") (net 7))
 (segment (start 224.22 105.8) (end 224.22 94.62) (width 0.25) (layer "F.Cu") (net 7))
 (segment (start 216.512 112.32) (end 215.756 113.076) (width 0.25) (layer "F.Cu") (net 7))
 (segment (start 206.44 111.84) (end 208.8 114.2) (width 0.25) (layer "F.Cu") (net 7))
 (segment (start 225.2 106.78) (end 224.22 105.8) (width 0.25) (layer "B.Cu") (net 7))
 (segment (start 225.2 111.75) (end 225.2 118.25) (width 0.25) (layer "B.Cu") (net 7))
 (segment (start 225.2 111.75) (end 225.2 106.78) (width 0.25) (layer "B.Cu") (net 7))
 (segment (start 221.68 103.33) (end 226.41 98.6) (width 0.25) (layer "B.Cu") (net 47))
 (segment (start 221.68 105.8) (end 221.68 103.33) (width 0.25) (layer "B.Cu") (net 47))
 (segment (start 203.976 95.424) (end 211.6 87.8) (width 0.25) (layer "B.Cu") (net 13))
 (segment (start 202.429 96.112884) (end 203.117884 95.424) (width 0.25) (layer "B.Cu") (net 13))
 (segment (start 203.117884 95.424) (end 203.976 95.424) (width 0.25) (layer "B.Cu") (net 13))
 (segment (start 202.429 100.504) (end 202.429 96.112884) (width 0.25) (layer "B.Cu") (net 13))
 (segment (start 203.605 101.68) (end 202.429 100.504) (width 0.25) (layer "B.Cu") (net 13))
 (segment (start 211.6 87.8) (end 211.6 87.08) (width 0.25) (layer "B.Cu") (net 13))
 (segment (start 212.776 100.267116) (end 212.776 90.796) (width 0.25) (layer "F.Cu") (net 12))
 (segment (start 208.823116 104.22) (end 212.776 100.267116) (width 0.25) (layer "F.Cu") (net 12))
 (segment (start 212.776 90.796) (end 211.6 89.62) (width 0.25) (layer "F.Cu") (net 12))
 (segment (start 203.605 104.22) (end 208.823116 104.22) (width 0.25) (layer "F.Cu") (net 12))
 (segment (start 203.605 96.6) (end 208.045 92.16) (width 0.25) (layer "B.Cu") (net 15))
 (segment (start 208.045 92.16) (end 211.6 92.16) (width 0.25) (layer "B.Cu") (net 15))
 (segment (start 181.4 59.8) (end 184.8 63.2) (width 0.25) (layer "F.Cu") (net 5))
 (segment (start 184.8 63.2) (end 184.8 63.68) (width 0.25) (layer "F.Cu") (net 5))
 (segment (start 184.8 63.68) (end 181.6 66.88) (width 0.25) (layer "B.Cu") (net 5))
 (segment (start 181.6 115.8) (end 182.72 116.92) (width 0.25) (layer "B.Cu") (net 5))
 (segment (start 182.72 116.92) (end 185.825 116.92) (width 0.25) (layer "B.Cu") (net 5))
 (segment (start 181.6 66.88) (end 181.6 115.8) (width 0.25) (layer "B.Cu") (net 5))
 (segment (start 204.085 114.86) (end 203.605 114.38) (width 0.25) (layer "F.Cu") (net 9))
 (segment (start 217 114.86) (end 204.085 114.86) (width 0.25) (layer "F.Cu") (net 9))
 (segment (start 217 117.4) (end 216.8 117.4) (width 0.25) (layer "F.Cu") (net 8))
 (segment (start 216.8 117.4) (end 216.32 116.92) (width 0.25) (layer "F.Cu") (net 8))
 (segment (start 216.32 116.92) (end 203.605 116.92) (width 0.25) (layer "F.Cu") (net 8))
 (segment (start 188.365 73.74) (end 185.825 76.28) (width 0.25) (layer "F.Cu") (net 30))
 (segment (start 185.825 78.82) (end 188.365 76.28) (width 0.25) (layer "F.Cu") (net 30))
 (segment (start 188.365 76.28) (end 188.365 73.74) (width 0.25) (layer "F.Cu") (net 30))
 (segment (start 188.365 63.6) (end 188.365 73.74) (width 0.25) (layer "F.Cu") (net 30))
 (segment (start 203.605 94.06) (end 210.96 94.06) (width 0.25) (layer "F.Cu") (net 16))
 (segment (start 210.96 94.06) (end 211.6 94.7) (width 0.25) (layer "F.Cu") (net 16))
 (segment (start 202.429 92.696) (end 202.429 95.236) (width 0.25) (layer "F.Cu") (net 17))
 (segment (start 202.429 95.236) (end 209.596 95.236) (width 0.25) (layer "F.Cu") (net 17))
 (segment (start 203.605 91.52) (end 202.429 92.696) (width 0.25) (layer "F.Cu") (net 17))
 (segment (start 209.596 95.236) (end 211.6 97.24) (width 0.25) (layer "F.Cu") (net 17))
 (segment (start 202.429 97.776) (end 209.596 97.776) (width 0.25) (layer "F.Cu") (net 18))
 (segment (start 201.978 90.607) (end 201.978 97.325) (width 0.25) (layer "F.Cu") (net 18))
 (segment (start 203.605 88.98) (end 201.978 90.607) (width 0.25) (layer "F.Cu") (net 18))
 (segment (start 201.978 97.325) (end 202.429 97.776) (width 0.25) (layer "F.Cu") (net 18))
 (segment (start 209.596 97.776) (end 211.6 99.78) (width 0.25) (layer "F.Cu") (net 18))
 (segment (start 214.35 105.4) (end 203.908116 105.4) (width 0.25) (layer "B.Cu") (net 6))
 (segment (start 203.908116 105.4) (end 203.904116 105.396) (width 0.25) (layer "B.Cu") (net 6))
 (segment (start 220.7 118.25) (end 220.7 111.75) (width 0.25) (layer "B.Cu") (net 6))
 (segment (start 199.701 105.396) (end 185.825 91.52) (width 0.25) (layer "B.Cu") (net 6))
 (segment (start 203.904116 105.396) (end 199.701 105.396) (width 0.25) (layer "B.Cu") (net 6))
 (segment (start 220.7 111.75) (end 214.35 105.4) (width 0.25) (layer "B.Cu") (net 6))
 (segment (start 193.445 99.14) (end 193.445 71.012) (width 0.25) (layer "F.Cu") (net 40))
 (segment (start 211.6 84.54) (end 207.056 79.996) (width 0.25) (layer "F.Cu") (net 40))
 (segment (start 193.445 71.012) (end 193.445 63.6) (width 0.25) (layer "F.Cu") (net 40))
 (segment (start 202.429 79.996) (end 193.445 71.012) (width 0.25) (layer "F.Cu") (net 40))
 (segment (start 207.056 79.996) (end 202.429 79.996) (width 0.25) (layer "F.Cu") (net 40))
 (segment (start 185.825 106.76) (end 193.445 99.14) (width 0.25) (layer "F.Cu") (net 40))
 (segment (start 218.79 98.6) (end 218.79 91.73) (width 0.25) (layer "B.Cu") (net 40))
 (segment (start 218.79 91.73) (end 211.6 84.54) (width 0.25) (layer "B.Cu") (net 40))
 (segment (start 212.8 59.33) (end 215.89 56.24) (width 0.25) (layer "F.Cu") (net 3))
 (segment (start 186.006 52.314) (end 184.8 53.52) (width 0.25) (layer "F.Cu") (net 3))
 (segment (start 192.319 52.314) (end 186.006 52.314) (width 0.25) (layer "F.Cu") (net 3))
 (segment (start 193.445 53.44) (end 195.605 55.6) (width 0.25) (layer "F.Cu") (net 3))
 (segment (start 212.8 70.45) (end 212.8 59.33) (width 0.25) (layer "F.Cu") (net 3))
 (segment (start 181.4 57.26) (end 181.4 56.92) (width 0.25) (layer "F.Cu") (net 3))
 (segment (start 215.25 55.6) (end 215.89 56.24) (width 0.25) (layer "F.Cu") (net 3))
 (segment (start 193.445 53.44) (end 192.319 52.314) (width 0.25) (layer "F.Cu") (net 3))
 (segment (start 209.4 55.6) (end 215.25 55.6) (width 0.25) (layer "F.Cu") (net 3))
 (segment (start 215.89 73.54) (end 212.8 70.45) (width 0.25) (layer "F.Cu") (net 3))
 (segment (start 181.4 56.92) (end 184.8 53.52) (width 0.25) (layer "F.Cu") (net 3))
 (segment (start 195.605 55.6) (end 209.4 55.6) (width 0.25) (layer "F.Cu") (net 3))
 (segment (start 209.4 63.22) (end 205.58 59.4) (width 0.25) (layer "F.Cu") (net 1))
 (segment (start 205.58 59.4) (end 194.325 59.4) (width 0.25) (layer "F.Cu") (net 1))
 (segment (start 194.325 59.4) (end 188.365 53.44) (width 0.25) (layer "F.Cu") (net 1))
 (segment (start 209.4 63.22) (end 218.43 72.25) (width 0.25) (layer "B.Cu") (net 1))
 (segment (start 218.43 56.24) (end 211.45 63.22) (width 0.25) (layer "B.Cu") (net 1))
 (segment (start 211.45 63.22) (end 209.4 63.22) (width 0.25) (layer "B.Cu") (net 1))
 (segment (start 218.43 72.25) (end 218.43 73.54) (width 0.25) (layer "B.Cu") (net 1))
 (segment (start 184.4 65.8) (end 182.4 67.8) (width 0.25) (layer "B.Cu") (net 42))
 (segment (start 182.4 111.2) (end 183.04 111.84) (width 0.25) (layer "B.Cu") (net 42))
 (segment (start 182.4 67.8) (end 182.4 111.2) (width 0.25) (layer "B.Cu") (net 42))
 (segment (start 195.985 63.6) (end 193.785 65.8) (width 0.25) (layer "B.Cu") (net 42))
 (segment (start 193.785 65.8) (end 184.4 65.8) (width 0.25) (layer "B.Cu") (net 42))
 (segment (start 183.04 111.84) (end 185.825 111.84) (width 0.25) (layer "B.Cu") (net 42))
 (segment (start 216.921 61.729) (end 215.89 62.76) (width 0.25) (layer "F.Cu") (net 4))
 (segment (start 197.225 52.2) (end 213.308055 52.2) (width 0.25) (layer "F.Cu") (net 4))
 (segment (start 213.308055 52.2) (end 216.921 55.812945) (width 0.25) (layer "F.Cu") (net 4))
 (segment (start 215.89 80.06) (end 217.399 78.551) (width 0.25) (layer "F.Cu") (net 4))
 (segment (start 215.89 82.09) (end 220.7 86.9) (width 0.25) (layer "F.Cu") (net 4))
 (segment (start 216.921 55.812945) (end 216.921 61.729) (width 0.25) (layer "F.Cu") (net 4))
 (segment (start 217.399 78.551) (end 217.399 64.269) (width 0.25) (layer "F.Cu") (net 4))
 (segment (start 195.985 53.44) (end 197.225 52.2) (width 0.25) (layer "F.Cu") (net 4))
 (segment (start 217.399 64.269) (end 215.89 62.76) (width 0.25) (layer "F.Cu") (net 4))
 (segment (start 215.89 80.06) (end 215.89 82.09) (width 0.25) (layer "F.Cu") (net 4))
 (segment (start 220.7 93.4) (end 220.7 86.9) (width 0.25) (layer "B.Cu") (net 4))
 (segment (start 223.6 73.4) (end 221 73.4) (width 0.25) (layer "F.Cu") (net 2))
 (segment (start 224.4 65.4) (end 224.4 72.6) (width 0.25) (layer "F.Cu") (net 2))
 (segment (start 221.76 62.76) (end 224.4 65.4) (width 0.25) (layer "F.Cu") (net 2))
 (segment (start 221.095908 80.06) (end 225.2 84.164092) (width 0.25) (layer "F.Cu") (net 2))
 (segment (start 225.2 84.164092) (end 225.2 86.9) (width 0.25) (layer "F.Cu") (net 2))
 (segment (start 218.43 62.76) (end 221.76 62.76) (width 0.25) (layer "F.Cu") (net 2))
 (segment (start 218.43 80.06) (end 221.095908 80.06) (width 0.25) (layer "F.Cu") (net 2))
 (segment (start 224.4 72.6) (end 223.6 73.4) (width 0.25) (layer "F.Cu") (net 2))
 (segment (start 218.43 75.97) (end 218.43 80.06) (width 0.25) (layer "F.Cu") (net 2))
 (segment (start 221 73.4) (end 218.43 75.97) (width 0.25) (layer "F.Cu") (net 2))
 (segment (start 225.2 93.4) (end 225.2 86.9) (width 0.25) (layer "B.Cu") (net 2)))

